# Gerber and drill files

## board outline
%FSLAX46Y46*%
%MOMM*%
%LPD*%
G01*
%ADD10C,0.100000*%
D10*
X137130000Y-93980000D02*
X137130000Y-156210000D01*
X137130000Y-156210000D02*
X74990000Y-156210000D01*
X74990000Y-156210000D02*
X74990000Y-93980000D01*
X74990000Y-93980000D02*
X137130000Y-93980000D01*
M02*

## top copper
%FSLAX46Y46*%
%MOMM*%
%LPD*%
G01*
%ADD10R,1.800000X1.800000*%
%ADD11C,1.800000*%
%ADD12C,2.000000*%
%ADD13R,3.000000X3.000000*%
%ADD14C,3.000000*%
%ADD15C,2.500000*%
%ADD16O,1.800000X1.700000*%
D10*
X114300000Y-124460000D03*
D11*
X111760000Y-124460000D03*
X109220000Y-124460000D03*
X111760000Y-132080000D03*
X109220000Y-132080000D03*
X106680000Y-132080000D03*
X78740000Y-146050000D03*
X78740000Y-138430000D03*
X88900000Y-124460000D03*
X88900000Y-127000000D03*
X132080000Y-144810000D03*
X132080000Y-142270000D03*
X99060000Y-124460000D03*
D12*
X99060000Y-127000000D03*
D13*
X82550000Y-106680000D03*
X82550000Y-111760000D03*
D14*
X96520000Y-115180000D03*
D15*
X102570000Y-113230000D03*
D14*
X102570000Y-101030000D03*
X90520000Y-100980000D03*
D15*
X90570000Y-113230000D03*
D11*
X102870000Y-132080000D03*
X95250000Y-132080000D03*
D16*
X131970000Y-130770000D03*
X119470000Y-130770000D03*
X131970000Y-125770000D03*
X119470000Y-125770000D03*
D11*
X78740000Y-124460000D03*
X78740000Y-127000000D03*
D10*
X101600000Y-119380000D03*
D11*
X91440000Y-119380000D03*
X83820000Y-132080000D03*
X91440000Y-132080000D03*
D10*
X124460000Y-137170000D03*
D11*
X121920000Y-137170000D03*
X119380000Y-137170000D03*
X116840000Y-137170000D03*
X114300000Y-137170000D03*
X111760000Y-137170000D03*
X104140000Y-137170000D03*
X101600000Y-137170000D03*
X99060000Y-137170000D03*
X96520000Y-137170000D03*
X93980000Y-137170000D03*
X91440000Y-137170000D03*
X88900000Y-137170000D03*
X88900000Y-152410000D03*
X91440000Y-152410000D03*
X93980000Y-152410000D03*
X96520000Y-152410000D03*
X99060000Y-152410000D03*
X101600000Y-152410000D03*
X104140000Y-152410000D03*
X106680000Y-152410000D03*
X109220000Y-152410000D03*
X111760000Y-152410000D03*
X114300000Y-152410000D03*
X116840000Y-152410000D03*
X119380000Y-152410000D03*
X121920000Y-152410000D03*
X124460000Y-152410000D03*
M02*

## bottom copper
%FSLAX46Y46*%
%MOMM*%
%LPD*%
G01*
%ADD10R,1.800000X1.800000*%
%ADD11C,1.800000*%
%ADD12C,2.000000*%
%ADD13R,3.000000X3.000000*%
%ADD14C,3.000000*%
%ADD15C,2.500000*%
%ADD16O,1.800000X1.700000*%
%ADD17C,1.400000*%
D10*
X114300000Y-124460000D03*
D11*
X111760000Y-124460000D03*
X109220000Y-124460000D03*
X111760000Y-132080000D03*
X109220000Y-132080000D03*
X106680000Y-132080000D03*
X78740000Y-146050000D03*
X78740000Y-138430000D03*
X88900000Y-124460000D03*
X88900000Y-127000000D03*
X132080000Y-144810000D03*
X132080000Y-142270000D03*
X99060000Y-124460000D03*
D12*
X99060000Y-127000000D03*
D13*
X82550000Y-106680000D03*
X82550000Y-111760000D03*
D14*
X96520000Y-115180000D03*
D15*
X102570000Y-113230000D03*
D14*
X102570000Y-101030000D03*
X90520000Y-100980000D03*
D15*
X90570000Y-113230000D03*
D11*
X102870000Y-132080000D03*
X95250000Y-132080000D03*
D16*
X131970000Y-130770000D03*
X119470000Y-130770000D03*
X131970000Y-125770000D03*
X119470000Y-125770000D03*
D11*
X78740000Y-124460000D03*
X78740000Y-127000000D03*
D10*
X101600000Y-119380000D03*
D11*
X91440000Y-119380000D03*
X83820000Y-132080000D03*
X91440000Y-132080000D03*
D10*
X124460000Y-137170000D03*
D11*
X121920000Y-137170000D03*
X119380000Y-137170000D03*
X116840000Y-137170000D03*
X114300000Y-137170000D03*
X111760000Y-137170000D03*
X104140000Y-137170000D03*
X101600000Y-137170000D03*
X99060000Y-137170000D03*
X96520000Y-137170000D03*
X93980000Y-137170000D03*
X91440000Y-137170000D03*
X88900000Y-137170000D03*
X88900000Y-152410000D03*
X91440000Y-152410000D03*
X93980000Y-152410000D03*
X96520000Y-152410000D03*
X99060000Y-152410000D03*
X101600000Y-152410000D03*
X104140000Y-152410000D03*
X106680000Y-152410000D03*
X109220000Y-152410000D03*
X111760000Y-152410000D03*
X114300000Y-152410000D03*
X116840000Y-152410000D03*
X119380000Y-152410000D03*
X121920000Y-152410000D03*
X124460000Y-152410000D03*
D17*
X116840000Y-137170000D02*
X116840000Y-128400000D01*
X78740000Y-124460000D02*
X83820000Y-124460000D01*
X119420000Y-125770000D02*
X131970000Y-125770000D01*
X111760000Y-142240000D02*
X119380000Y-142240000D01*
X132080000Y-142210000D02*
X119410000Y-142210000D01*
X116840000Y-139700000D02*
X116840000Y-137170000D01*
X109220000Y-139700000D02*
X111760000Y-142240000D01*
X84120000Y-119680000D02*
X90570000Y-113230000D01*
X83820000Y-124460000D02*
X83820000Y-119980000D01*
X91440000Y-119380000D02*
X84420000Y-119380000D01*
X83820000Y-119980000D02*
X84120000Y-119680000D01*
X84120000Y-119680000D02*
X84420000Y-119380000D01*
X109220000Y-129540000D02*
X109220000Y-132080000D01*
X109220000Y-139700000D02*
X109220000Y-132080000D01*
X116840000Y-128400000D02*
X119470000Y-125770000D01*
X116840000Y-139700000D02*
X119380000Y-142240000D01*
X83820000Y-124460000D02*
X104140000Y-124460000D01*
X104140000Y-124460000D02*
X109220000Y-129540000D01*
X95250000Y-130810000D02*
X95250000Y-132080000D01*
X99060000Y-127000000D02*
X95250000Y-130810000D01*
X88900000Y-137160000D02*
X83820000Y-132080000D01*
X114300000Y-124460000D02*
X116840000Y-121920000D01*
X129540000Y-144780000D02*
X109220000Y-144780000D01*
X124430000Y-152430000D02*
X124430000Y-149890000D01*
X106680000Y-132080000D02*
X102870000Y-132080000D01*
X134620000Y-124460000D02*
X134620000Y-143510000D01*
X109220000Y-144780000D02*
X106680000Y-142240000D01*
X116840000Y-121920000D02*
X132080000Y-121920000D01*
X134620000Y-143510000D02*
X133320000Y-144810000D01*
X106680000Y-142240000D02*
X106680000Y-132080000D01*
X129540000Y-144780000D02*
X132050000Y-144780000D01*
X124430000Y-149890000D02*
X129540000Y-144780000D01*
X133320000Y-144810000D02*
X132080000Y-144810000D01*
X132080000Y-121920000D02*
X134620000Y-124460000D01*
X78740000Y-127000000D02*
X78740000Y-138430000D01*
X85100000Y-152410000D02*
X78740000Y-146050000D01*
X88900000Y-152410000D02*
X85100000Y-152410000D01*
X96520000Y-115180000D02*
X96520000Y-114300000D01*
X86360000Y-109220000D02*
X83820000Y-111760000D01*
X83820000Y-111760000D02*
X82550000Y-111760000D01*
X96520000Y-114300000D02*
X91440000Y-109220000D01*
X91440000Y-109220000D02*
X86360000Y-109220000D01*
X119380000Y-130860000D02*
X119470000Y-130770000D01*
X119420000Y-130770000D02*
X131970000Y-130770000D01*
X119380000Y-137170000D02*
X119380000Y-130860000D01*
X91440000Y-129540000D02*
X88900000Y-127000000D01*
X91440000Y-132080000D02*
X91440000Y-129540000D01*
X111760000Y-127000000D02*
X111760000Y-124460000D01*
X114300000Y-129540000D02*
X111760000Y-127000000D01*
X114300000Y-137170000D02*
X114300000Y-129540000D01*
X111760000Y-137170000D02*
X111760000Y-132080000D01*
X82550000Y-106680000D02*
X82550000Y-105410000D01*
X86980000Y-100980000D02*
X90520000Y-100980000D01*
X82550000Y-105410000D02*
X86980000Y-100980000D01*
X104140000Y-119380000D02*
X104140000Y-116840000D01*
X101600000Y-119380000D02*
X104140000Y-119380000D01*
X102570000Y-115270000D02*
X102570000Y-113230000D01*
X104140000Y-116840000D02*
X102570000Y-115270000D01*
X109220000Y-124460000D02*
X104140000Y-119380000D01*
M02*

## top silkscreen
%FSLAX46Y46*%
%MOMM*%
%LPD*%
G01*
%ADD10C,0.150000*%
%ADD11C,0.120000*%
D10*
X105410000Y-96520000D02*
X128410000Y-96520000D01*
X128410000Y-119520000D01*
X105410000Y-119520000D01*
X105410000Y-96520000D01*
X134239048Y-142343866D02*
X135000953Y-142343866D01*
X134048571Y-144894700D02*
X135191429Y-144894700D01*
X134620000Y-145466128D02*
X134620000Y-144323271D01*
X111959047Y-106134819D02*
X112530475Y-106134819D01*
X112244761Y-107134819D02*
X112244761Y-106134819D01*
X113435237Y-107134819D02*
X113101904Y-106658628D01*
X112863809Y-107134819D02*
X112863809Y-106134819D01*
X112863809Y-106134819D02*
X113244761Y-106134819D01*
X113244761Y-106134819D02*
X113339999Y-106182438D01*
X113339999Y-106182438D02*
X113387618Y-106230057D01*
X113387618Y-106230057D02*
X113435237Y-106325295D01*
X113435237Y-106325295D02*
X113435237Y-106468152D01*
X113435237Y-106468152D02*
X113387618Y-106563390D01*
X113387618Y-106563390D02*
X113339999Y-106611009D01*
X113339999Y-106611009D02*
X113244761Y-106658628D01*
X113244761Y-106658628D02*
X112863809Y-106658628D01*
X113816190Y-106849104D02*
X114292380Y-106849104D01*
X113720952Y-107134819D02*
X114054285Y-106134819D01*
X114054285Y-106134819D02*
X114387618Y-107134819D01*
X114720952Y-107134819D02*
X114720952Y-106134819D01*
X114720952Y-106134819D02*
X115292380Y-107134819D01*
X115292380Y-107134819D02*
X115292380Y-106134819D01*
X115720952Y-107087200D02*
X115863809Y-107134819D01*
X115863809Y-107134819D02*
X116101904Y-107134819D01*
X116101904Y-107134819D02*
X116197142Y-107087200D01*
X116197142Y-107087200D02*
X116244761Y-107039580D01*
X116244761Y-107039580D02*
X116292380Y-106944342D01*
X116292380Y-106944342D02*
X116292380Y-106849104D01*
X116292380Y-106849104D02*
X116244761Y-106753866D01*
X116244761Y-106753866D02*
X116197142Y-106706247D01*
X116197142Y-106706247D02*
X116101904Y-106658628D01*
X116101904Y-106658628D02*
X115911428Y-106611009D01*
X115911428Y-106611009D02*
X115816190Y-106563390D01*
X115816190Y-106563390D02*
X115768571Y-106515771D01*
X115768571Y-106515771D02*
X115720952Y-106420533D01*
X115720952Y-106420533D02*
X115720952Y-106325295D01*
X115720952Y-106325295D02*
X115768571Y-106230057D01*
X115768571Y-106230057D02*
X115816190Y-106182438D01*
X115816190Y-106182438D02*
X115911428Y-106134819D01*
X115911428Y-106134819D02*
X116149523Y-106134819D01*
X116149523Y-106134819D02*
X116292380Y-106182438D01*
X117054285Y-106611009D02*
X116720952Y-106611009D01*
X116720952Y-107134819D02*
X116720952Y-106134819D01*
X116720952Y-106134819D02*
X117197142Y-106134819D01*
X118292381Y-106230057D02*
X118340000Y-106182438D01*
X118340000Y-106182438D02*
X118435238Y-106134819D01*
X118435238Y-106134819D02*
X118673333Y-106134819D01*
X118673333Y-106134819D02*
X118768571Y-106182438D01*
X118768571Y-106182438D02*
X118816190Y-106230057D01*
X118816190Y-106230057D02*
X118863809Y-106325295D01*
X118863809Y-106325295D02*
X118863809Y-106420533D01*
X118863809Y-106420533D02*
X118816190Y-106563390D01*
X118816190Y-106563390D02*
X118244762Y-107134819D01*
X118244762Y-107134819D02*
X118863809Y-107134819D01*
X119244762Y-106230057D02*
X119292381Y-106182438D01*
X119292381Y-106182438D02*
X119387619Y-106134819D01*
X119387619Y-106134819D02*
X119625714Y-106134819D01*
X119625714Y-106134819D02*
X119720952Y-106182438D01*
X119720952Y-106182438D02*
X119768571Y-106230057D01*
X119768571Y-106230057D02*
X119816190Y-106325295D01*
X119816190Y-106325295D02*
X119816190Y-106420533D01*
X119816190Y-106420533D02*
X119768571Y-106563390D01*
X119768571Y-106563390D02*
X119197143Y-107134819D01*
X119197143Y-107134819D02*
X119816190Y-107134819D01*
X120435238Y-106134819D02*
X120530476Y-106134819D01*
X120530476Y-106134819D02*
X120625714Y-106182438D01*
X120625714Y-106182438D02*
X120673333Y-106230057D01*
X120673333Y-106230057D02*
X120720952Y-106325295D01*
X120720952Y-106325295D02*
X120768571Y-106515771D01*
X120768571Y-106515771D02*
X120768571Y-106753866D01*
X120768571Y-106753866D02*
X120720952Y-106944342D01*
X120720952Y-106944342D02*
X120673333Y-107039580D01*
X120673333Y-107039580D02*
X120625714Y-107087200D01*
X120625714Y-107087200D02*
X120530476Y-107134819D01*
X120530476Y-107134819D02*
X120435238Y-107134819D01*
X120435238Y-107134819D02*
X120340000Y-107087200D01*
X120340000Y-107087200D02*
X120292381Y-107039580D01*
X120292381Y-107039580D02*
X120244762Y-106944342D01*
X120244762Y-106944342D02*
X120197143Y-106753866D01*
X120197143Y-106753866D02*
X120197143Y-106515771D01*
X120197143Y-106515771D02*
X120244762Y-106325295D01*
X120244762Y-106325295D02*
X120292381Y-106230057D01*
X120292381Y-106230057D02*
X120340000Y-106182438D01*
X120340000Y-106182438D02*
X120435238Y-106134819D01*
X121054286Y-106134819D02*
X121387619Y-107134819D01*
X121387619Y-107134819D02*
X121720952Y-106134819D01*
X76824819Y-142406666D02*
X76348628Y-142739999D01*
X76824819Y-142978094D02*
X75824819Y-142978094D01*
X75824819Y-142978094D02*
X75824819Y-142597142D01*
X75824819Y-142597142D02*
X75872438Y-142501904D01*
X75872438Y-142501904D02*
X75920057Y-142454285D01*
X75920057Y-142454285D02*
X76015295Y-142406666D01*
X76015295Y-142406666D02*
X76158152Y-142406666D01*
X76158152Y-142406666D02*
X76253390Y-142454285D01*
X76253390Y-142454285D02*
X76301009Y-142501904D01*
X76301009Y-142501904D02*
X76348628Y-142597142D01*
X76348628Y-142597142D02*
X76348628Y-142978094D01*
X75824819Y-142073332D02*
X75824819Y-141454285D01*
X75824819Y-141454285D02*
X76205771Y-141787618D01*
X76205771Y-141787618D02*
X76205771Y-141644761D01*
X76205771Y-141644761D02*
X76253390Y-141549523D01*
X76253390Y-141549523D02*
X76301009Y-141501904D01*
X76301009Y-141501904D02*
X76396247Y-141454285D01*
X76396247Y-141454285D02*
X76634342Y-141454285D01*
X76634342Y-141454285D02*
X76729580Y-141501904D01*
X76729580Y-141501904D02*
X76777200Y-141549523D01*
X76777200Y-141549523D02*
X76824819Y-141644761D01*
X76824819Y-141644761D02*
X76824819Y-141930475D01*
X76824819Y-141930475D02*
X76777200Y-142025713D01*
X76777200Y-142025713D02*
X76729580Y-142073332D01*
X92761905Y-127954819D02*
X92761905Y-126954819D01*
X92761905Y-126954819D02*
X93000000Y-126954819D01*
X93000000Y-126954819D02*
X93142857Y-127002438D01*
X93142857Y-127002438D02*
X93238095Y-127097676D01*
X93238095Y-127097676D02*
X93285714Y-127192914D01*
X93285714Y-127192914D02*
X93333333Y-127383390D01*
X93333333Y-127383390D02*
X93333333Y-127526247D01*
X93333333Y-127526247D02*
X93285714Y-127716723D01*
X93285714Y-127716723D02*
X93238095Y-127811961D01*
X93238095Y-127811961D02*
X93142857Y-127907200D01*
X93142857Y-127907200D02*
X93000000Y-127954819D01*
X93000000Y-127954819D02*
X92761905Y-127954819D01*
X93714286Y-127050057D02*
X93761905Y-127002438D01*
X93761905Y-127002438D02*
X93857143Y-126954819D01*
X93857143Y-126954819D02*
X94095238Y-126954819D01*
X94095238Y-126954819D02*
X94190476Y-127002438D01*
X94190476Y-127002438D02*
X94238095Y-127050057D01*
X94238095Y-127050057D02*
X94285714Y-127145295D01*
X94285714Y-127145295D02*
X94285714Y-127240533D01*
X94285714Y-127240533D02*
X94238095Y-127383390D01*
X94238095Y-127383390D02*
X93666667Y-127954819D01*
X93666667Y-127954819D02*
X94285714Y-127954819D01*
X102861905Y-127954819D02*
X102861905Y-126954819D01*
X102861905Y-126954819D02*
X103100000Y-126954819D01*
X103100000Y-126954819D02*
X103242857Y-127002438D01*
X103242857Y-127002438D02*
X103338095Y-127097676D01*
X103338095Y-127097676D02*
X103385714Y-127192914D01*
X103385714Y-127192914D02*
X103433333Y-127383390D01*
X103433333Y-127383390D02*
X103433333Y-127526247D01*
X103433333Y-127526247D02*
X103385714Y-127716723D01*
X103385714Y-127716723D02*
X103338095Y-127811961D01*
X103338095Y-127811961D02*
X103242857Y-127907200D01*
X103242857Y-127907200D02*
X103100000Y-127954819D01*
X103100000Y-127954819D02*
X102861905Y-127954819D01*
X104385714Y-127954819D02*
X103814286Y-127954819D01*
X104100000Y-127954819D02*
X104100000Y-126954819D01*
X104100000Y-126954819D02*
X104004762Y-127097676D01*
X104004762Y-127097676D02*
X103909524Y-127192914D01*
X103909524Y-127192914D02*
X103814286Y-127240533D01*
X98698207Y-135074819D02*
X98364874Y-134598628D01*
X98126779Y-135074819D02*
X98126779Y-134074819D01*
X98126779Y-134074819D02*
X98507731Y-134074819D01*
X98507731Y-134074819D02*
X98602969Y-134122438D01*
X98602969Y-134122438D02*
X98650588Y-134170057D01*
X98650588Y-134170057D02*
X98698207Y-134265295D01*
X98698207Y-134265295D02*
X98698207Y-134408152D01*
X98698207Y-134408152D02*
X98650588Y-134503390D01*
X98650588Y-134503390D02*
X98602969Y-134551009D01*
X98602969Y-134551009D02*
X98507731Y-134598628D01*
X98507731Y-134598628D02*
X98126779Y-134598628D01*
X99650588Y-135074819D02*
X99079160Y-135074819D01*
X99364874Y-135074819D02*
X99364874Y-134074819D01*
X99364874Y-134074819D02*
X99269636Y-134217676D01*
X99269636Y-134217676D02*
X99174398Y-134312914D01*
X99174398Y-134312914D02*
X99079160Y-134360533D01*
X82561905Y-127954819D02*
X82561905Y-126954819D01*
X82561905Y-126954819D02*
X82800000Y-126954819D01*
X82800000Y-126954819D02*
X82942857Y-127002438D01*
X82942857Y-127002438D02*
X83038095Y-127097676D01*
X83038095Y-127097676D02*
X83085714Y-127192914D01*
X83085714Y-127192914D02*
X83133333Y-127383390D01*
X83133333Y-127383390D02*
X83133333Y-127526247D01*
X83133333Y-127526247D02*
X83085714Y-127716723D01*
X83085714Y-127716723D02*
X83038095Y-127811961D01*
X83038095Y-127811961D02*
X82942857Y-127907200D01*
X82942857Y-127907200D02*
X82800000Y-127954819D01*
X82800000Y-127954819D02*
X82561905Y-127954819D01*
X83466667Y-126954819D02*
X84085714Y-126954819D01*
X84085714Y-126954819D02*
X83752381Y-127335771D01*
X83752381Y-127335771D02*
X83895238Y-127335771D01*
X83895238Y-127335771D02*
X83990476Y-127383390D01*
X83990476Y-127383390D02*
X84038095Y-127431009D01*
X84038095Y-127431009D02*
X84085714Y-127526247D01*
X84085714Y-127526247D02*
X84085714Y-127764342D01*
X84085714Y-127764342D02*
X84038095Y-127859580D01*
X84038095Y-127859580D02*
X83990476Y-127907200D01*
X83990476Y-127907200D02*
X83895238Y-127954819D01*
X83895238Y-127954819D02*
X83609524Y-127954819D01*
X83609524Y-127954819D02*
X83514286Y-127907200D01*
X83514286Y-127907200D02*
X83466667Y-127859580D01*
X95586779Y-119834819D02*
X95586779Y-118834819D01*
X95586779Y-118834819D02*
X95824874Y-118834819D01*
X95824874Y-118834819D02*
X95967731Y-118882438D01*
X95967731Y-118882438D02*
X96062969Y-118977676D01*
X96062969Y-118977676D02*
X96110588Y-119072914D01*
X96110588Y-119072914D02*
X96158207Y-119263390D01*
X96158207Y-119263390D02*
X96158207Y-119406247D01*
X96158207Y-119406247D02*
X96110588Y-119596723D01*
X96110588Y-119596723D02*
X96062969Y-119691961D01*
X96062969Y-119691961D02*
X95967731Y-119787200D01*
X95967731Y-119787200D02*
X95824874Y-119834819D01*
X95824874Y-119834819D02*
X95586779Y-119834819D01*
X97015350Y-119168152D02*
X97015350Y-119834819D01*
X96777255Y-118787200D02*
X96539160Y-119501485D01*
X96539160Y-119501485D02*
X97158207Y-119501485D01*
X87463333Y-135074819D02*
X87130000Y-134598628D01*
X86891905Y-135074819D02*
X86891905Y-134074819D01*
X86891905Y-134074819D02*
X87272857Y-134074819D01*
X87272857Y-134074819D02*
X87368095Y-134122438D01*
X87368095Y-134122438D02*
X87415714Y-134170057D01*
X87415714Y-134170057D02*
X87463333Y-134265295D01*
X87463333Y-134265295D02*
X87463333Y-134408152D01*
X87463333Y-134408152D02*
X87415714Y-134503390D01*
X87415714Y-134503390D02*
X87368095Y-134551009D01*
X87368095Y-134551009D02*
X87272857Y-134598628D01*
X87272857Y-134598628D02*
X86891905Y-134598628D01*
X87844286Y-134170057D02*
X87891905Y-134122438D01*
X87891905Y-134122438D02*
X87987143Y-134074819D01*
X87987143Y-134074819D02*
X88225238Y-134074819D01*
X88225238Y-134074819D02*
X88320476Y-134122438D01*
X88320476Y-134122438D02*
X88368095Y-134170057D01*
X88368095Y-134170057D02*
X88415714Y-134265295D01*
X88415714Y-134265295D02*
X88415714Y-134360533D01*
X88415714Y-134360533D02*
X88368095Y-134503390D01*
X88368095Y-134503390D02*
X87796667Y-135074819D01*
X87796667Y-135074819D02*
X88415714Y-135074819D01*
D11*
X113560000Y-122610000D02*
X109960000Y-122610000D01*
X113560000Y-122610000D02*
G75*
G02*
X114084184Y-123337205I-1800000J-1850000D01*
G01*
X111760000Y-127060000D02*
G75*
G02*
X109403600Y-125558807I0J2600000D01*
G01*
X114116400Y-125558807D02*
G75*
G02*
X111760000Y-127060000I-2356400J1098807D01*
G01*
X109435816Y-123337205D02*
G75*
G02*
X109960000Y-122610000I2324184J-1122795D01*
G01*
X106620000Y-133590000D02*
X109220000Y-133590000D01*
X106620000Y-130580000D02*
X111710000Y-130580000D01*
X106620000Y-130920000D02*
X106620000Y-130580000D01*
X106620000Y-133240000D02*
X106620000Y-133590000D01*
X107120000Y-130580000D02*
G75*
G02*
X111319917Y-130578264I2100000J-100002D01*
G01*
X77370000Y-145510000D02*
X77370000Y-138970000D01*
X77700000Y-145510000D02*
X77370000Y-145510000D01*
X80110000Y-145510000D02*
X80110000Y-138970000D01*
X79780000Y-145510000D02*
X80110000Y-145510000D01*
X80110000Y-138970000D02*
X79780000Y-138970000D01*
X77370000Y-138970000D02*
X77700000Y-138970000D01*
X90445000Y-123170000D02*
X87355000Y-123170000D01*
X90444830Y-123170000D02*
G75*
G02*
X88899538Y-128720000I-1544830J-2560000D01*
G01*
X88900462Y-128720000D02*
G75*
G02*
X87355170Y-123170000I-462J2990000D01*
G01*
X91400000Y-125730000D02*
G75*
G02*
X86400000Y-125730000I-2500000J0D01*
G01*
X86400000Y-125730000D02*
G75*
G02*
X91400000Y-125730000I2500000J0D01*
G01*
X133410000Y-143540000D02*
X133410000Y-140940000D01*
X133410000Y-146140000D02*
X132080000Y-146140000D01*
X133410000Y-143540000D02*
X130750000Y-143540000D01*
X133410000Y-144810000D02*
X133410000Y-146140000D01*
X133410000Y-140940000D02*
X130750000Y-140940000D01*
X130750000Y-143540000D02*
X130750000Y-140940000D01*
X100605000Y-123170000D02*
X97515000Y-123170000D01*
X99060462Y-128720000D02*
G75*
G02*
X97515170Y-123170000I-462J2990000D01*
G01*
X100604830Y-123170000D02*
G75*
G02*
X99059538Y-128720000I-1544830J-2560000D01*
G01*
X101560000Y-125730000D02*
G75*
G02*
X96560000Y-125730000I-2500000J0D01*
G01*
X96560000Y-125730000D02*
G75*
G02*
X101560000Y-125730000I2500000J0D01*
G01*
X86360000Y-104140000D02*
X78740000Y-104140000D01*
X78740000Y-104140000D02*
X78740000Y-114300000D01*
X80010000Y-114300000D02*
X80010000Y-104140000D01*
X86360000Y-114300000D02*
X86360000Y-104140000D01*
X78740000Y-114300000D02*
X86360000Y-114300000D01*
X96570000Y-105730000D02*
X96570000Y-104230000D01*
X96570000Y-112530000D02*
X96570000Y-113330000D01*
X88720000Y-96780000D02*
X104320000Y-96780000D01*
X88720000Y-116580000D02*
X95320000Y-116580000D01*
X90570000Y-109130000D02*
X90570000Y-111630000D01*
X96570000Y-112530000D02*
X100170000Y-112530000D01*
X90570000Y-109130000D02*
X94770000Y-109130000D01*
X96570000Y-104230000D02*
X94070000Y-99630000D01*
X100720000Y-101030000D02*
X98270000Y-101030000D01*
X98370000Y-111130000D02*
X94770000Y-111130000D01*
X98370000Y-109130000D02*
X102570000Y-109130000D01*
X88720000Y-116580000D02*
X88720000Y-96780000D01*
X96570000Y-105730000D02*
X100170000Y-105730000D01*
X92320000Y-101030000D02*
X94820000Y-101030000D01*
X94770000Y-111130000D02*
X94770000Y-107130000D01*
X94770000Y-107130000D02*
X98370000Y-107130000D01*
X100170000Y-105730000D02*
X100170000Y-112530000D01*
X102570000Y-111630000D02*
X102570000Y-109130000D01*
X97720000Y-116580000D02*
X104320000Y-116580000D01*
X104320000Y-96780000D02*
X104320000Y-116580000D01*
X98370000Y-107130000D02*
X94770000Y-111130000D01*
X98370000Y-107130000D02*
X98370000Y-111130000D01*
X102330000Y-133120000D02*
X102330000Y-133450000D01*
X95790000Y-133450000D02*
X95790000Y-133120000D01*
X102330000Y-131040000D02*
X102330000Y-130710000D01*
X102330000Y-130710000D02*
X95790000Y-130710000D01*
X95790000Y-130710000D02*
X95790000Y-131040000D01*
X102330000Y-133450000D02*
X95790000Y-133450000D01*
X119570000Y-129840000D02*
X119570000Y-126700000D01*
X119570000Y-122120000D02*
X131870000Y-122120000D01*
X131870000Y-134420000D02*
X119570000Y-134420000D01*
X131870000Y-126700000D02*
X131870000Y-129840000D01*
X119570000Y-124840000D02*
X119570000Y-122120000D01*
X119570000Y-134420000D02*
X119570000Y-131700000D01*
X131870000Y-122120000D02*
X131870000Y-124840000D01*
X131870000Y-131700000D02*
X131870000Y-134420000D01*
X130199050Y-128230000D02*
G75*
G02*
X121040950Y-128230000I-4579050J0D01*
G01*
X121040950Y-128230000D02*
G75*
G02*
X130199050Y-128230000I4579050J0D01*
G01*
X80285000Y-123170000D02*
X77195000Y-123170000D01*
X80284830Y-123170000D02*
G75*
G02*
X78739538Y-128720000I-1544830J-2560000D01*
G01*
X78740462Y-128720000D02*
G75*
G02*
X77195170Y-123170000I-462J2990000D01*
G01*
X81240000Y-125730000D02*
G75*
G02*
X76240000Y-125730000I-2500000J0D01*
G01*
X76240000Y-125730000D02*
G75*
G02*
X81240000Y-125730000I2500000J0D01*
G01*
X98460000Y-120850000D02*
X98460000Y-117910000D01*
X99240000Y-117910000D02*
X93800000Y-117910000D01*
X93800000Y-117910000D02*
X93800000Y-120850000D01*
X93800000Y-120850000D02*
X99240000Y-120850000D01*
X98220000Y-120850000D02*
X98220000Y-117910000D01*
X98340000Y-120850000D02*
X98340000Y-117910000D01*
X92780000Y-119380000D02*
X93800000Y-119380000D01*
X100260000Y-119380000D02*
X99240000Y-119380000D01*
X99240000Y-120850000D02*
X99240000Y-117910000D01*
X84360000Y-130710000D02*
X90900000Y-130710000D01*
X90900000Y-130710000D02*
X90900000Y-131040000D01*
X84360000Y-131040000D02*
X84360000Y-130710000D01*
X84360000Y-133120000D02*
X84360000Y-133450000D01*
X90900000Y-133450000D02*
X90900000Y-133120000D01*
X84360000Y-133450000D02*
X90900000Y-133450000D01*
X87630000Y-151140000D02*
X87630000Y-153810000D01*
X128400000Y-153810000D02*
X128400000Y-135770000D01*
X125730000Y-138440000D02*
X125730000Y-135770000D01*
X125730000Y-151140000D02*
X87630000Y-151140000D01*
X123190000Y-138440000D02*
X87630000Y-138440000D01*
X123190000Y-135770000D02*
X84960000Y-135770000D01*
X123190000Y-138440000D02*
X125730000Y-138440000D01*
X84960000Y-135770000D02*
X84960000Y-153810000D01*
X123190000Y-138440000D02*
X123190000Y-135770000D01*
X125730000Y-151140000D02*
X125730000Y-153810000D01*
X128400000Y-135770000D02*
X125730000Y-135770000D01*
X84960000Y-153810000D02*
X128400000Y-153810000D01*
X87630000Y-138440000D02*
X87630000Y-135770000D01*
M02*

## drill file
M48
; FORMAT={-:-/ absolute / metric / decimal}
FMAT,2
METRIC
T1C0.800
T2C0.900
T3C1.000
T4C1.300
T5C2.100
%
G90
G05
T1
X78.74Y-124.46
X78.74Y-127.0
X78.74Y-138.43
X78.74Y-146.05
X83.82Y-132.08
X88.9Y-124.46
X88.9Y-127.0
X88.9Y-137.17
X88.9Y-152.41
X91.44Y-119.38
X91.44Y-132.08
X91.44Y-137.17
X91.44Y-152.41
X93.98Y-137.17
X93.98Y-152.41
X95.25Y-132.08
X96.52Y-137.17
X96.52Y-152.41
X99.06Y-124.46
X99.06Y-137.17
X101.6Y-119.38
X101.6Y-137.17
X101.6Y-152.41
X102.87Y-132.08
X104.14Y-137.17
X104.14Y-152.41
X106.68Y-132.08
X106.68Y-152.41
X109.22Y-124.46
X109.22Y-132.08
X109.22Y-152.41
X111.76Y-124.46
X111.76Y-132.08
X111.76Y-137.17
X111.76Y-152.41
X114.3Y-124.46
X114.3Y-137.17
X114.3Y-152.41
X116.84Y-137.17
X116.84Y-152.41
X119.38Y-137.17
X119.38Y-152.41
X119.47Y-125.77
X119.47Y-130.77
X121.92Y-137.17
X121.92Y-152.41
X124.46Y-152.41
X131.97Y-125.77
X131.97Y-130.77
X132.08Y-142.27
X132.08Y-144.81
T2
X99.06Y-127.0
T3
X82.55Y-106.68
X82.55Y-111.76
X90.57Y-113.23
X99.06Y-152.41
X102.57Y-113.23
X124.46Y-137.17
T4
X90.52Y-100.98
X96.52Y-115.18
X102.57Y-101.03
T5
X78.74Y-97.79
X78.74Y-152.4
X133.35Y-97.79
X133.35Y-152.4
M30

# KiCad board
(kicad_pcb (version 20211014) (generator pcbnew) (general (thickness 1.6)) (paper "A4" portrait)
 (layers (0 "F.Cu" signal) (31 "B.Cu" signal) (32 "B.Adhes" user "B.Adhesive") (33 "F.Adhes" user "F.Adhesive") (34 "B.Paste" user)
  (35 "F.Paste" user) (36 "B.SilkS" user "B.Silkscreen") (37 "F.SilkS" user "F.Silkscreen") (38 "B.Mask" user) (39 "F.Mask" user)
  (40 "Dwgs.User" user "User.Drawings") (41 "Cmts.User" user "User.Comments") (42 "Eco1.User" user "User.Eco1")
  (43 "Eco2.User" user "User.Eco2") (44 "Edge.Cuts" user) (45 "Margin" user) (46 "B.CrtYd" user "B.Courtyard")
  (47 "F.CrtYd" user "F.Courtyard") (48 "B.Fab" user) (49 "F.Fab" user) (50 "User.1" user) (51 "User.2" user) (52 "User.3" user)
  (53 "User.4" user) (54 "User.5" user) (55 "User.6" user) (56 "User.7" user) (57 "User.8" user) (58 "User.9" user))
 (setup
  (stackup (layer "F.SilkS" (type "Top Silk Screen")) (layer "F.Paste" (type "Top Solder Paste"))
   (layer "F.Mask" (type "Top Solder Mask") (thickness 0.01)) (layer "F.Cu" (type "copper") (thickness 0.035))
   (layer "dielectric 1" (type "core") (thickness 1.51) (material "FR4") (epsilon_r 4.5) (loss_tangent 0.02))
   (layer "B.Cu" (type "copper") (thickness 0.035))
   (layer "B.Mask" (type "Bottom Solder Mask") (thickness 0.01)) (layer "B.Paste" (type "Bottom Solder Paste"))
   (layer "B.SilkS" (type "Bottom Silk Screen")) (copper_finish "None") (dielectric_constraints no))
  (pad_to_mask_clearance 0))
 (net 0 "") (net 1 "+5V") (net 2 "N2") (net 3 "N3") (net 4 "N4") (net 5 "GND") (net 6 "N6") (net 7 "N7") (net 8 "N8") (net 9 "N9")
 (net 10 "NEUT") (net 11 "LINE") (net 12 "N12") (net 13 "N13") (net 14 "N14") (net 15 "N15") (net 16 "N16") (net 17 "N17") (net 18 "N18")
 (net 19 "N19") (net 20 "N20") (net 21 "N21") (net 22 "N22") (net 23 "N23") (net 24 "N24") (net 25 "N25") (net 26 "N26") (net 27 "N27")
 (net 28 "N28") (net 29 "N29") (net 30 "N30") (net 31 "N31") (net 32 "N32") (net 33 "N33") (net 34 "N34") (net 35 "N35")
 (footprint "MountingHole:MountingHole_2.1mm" (layer "F.Cu") (at 133.35 97.79)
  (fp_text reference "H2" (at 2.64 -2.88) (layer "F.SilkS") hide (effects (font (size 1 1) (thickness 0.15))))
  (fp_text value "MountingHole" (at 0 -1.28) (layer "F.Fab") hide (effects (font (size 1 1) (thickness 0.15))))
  (pad "" np_thru_hole circle (at 0 0) (size 2.1 2.1) (drill 2.1) (layers *.Cu *.Mask)))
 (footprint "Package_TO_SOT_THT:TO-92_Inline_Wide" (layer "F.Cu") (at 114.3 124.46 180)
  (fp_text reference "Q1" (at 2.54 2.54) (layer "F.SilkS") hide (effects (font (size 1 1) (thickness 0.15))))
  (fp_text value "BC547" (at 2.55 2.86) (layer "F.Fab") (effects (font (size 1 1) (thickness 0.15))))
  (fp_line (start 0.74 1.85) (end 4.34 1.85) (layer "F.SilkS") (width 0.12))
  (fp_arc (start 0.74 1.85) (mid 0.446097 1.509328) (end 0.215816 1.122795) (layer "F.SilkS") (width 0.12))
  (fp_arc (start 2.54 -2.6) (mid 3.936979 -2.192818) (end 4.8964 -1.098807) (layer "F.SilkS") (width 0.12))
  (fp_arc (start 0.1836 -1.098807) (mid 1.143021 -2.192817) (end 2.54 -2.6) (layer "F.SilkS") (width 0.12))
  (fp_arc (start 4.864184 1.122795) (mid 4.633903 1.509328) (end 4.34 1.85) (layer "F.SilkS") (width 0.12))
  (pad "1" thru_hole rect (at 0 0 180) (size 1.8 1.8) (drill 0.8) (layers *.Cu *.Mask) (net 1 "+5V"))
  (pad "2" thru_hole circle (at 2.54 0 180) (size 1.8 1.8) (drill 0.8) (layers *.Cu *.Mask) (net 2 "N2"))
  (pad "3" thru_hole circle (at 5.08 0 180) (size 1.8 1.8) (drill 0.8) (layers *.Cu *.Mask) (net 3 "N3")))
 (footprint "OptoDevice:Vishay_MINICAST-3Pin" (layer "F.Cu") (at 111.76 132.08 180)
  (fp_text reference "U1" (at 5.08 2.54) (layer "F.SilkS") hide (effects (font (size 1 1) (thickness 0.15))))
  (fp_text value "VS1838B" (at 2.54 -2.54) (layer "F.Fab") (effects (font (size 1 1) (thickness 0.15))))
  (fp_line (start 5.14 -1.51) (end 2.54 -1.51) (layer "F.SilkS") (width 0.12))
  (fp_line (start 5.14 1.5) (end 0.05 1.5) (layer "F.SilkS") (width 0.12))
  (fp_line (start 5.14 1.16) (end 5.14 1.5) (layer "F.SilkS") (width 0.12))
  (fp_line (start 5.14 -1.16) (end 5.14 -1.51) (layer "F.SilkS") (width 0.12))
  (fp_arc (start 4.64 1.5) (mid 2.540869 3.502378) (end 0.440083 1.501736) (layer "F.SilkS") (width 0.12))
  (pad "1" thru_hole circle (at 0 0 180) (size 1.8 1.8) (drill 0.8) (layers *.Cu *.Mask) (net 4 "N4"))
  (pad "2" thru_hole circle (at 2.54 0 180) (size 1.8 1.8) (drill 0.8) (layers *.Cu *.Mask) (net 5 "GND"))
  (pad "3" thru_hole circle (at 5.08 0 180) (size 1.8 1.8) (drill 0.8) (layers *.Cu *.Mask) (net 1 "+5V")))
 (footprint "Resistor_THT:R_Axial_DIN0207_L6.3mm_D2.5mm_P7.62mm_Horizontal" (layer "F.Cu") (at 78.74 146.05 90)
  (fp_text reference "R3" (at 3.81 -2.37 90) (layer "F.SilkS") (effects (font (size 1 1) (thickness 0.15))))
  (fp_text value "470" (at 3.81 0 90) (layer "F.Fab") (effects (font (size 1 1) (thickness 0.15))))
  (fp_line (start 0.54 -1.37) (end 7.08 -1.37) (layer "F.SilkS") (width 0.12))
  (fp_line (start 0.54 -1.04) (end 0.54 -1.37) (layer "F.SilkS") (width 0.12))
  (fp_line (start 0.54 1.37) (end 7.08 1.37) (layer "F.SilkS") (width 0.12))
  (fp_line (start 0.54 1.04) (end 0.54 1.37) (layer "F.SilkS") (width 0.12))
  (fp_line (start 7.08 1.37) (end 7.08 1.04) (layer "F.SilkS") (width 0.12))
  (fp_line (start 7.08 -1.37) (end 7.08 -1.04) (layer "F.SilkS") (width 0.12))
  (pad "1" thru_hole circle (at 0 0 90) (size 1.8 1.8) (drill 0.8) (layers *.Cu *.Mask) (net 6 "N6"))
  (pad "2" thru_hole circle (at 7.62 0 90) (size 1.8 1.8) (drill 0.8) (layers *.Cu *.Mask) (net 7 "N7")))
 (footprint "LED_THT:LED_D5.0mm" (layer "F.Cu") (at 88.9 124.46 -90)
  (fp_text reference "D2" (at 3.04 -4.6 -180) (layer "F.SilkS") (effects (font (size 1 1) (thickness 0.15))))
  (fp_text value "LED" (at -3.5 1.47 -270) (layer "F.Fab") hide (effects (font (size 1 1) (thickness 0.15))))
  (fp_line (start -1.29 -1.545) (end -1.29 1.545) (layer "F.SilkS") (width 0.12))
  (fp_arc (start -1.29 -1.54483) (mid 2.072002 -2.880433) (end 4.26 0.000462) (layer "F.SilkS") (width 0.12))
  (fp_arc (start 4.26 -0.000462) (mid 2.072002 2.880433) (end -1.29 1.54483) (layer "F.SilkS") (width 0.12))
  (fp_circle (center 1.27 0) (end 3.77 0) (layer "F.SilkS") (width 0.12) (fill none))
  (pad "1" thru_hole circle (at 0 0 270) (size 1.8 1.8) (drill 0.8) (layers *.Cu *.Mask) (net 5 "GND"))
  (pad "2" thru_hole circle (at 2.54 0 270) (size 1.8 1.8) (drill 0.8) (layers *.Cu *.Mask) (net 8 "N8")))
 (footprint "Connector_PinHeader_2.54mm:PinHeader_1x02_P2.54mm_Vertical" (layer "F.Cu") (at 132.08 144.81 180)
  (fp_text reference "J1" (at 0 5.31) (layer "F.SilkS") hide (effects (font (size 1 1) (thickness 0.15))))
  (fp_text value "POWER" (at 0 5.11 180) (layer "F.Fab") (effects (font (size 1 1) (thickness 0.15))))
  (fp_line (start -1.33 1.27) (end -1.33 3.87) (layer "F.SilkS") (width 0.12))
  (fp_line (start -1.33 -1.33) (end 0 -1.33) (layer "F.SilkS") (width 0.12))
  (fp_line (start -1.33 1.27) (end 1.33 1.27) (layer "F.SilkS") (width 0.12))
  (fp_line (start -1.33 0) (end -1.33 -1.33) (layer "F.SilkS") (width 0.12))
  (fp_line (start -1.33 3.87) (end 1.33 3.87) (layer "F.SilkS") (width 0.12))
  (fp_line (start 1.33 1.27) (end 1.33 3.87) (layer "F.SilkS") (width 0.12))
  (pad "1" thru_hole circle (at 0 0 180) (size 1.8 1.8) (drill 0.8) (layers *.Cu *.Mask) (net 1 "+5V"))
  (pad "2" thru_hole circle (at 0 2.54 180) (size 1.8 1.8) (drill 0.8) (layers *.Cu *.Mask) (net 5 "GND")))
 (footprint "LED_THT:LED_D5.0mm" (layer "F.Cu") (at 99.06 124.46 -90)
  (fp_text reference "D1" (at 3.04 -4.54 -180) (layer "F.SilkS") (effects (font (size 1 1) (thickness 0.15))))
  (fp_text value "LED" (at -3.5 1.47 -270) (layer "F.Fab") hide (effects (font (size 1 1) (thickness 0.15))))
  (fp_line (start -1.29 -1.545) (end -1.29 1.545) (layer "F.SilkS") (width 0.12))
  (fp_arc (start 4.26 -0.000462) (mid 2.072002 2.880433) (end -1.29 1.54483) (layer "F.SilkS") (width 0.12))
  (fp_arc (start -1.29 -1.54483) (mid 2.072002 -2.880433) (end 4.26 0.000462) (layer "F.SilkS") (width 0.12))
  (fp_circle (center 1.27 0) (end 3.77 0) (layer "F.SilkS") (width 0.12) (fill none))
  (pad "1" thru_hole circle (at 0 0 270) (size 1.8 1.8) (drill 0.8) (layers *.Cu *.Mask) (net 5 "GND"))
  (pad "2" thru_hole circle (at 2.54 0 270) (size 2 2) (drill 0.9) (layers *.Cu *.Mask) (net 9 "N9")))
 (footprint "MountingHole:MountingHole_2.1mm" (layer "F.Cu") (at 133.35 152.4)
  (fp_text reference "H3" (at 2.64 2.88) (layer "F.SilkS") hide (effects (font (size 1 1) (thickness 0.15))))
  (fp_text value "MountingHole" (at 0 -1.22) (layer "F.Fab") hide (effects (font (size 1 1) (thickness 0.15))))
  (pad "" np_thru_hole circle (at 0 0) (size 2.1 2.1) (drill 2.1) (layers *.Cu *.Mask)))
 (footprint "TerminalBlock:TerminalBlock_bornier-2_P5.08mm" (layer "F.Cu") (at 82.55 106.68 -90)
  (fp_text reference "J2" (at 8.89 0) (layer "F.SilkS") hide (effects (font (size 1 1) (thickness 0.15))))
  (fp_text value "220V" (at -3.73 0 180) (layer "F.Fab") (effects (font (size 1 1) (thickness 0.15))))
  (fp_line (start -2.54 -3.81) (end -2.54 3.81) (layer "F.SilkS") (width 0.12))
  (fp_line (start -2.54 3.81) (end 7.62 3.81) (layer "F.SilkS") (width 0.12))
  (fp_line (start 7.62 2.54) (end -2.54 2.54) (layer "F.SilkS") (width 0.12))
  (fp_line (start 7.62 -3.81) (end -2.54 -3.81) (layer "F.SilkS") (width 0.12))
  (fp_line (start 7.62 3.81) (end 7.62 -3.81) (layer "F.SilkS") (width 0.12))
  (pad "1" thru_hole rect (at 0 0 270) (size 3 3) (drill 1) (layers *.Cu *.Mask) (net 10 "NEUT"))
  (pad "2" thru_hole rect (at 5.08 0 270) (size 3 3) (drill 1) (layers *.Cu *.Mask) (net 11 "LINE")))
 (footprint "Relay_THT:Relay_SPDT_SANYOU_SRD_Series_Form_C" (layer "F.Cu") (at 96.52 115.18 90)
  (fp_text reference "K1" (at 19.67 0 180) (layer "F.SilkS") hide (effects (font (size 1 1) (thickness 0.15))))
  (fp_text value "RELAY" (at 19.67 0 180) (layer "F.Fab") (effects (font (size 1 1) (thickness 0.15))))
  (fp_line (start 9.45 0.05) (end 10.95 0.05) (layer "F.SilkS") (width 0.12))
  (fp_line (start 2.65 0.05) (end 1.85 0.05) (layer "F.SilkS") (width 0.12))
  (fp_line (start 18.4 -7.8) (end 18.4 7.8) (layer "F.SilkS") (width 0.12))
  (fp_line (start -1.4 -7.8) (end -1.4 -1.2) (layer "F.SilkS") (width 0.12))
  (fp_line (start 6.05 -5.95) (end 3.55 -5.95) (layer "F.SilkS") (width 0.12))
  (fp_line (start 2.65 0.05) (end 2.65 3.65) (layer "F.SilkS") (width 0.12))
  (fp_line (start 6.05 -5.95) (end 6.05 -1.75) (layer "F.SilkS") (width 0.12))
  (fp_line (start 10.95 0.05) (end 15.55 -2.45) (layer "F.SilkS") (width 0.12))
  (fp_line (start 14.15 4.2) (end 14.15 1.75) (layer "F.SilkS") (width 0.12))
  (fp_line (start 4.05 1.85) (end 4.05 -1.75) (layer "F.SilkS") (width 0.12))
  (fp_line (start 6.05 1.85) (end 6.05 6.05) (layer "F.SilkS") (width 0.12))
  (fp_line (start -1.4 -7.8) (end 18.4 -7.8) (layer "F.SilkS") (width 0.12))
  (fp_line (start 9.45 0.05) (end 9.45 3.65) (layer "F.SilkS") (width 0.12))
  (fp_line (start 14.15 -4.2) (end 14.15 -1.7) (layer "F.SilkS") (width 0.12))
  (fp_line (start 4.05 -1.75) (end 8.05 -1.75) (layer "F.SilkS") (width 0.12))
  (fp_line (start 8.05 -1.75) (end 8.05 1.85) (layer "F.SilkS") (width 0.12))
  (fp_line (start 9.45 3.65) (end 2.65 3.65) (layer "F.SilkS") (width 0.12))
  (fp_line (start 3.55 6.05) (end 6.05 6.05) (layer "F.SilkS") (width 0.12))
  (fp_line (start -1.4 1.2) (end -1.4 7.8) (layer "F.SilkS") (width 0.12))
  (fp_line (start 18.4 7.8) (end -1.4 7.8) (layer "F.SilkS") (width 0.12))
  (fp_line (start 8.05 1.85) (end 4.05 -1.75) (layer "F.SilkS") (width 0.12))
  (fp_line (start 8.05 1.85) (end 4.05 1.85) (layer "F.SilkS") (width 0.12))
  (pad "1" thru_hole circle (at 0 0 180) (size 3 3) (drill 1.3) (layers *.Cu *.Mask) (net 11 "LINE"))
  (pad "2" thru_hole circle (at 1.95 6.05 180) (size 2.5 2.5) (drill 1) (layers *.Cu *.Mask) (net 3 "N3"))
  (pad "3" thru_hole circle (at 14.15 6.05 180) (size 3 3) (drill 1.3) (layers *.Cu *.Mask) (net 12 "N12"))
  (pad "4" thru_hole circle (at 14.2 -6 180) (size 3 3) (drill 1.3) (layers *.Cu *.Mask) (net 10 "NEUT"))
  (pad "5" thru_hole circle (at 1.95 -5.95 180) (size 2.5 2.5) (drill 1) (layers *.Cu *.Mask) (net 5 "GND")))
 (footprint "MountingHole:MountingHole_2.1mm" (layer "F.Cu") (at 78.74 152.4)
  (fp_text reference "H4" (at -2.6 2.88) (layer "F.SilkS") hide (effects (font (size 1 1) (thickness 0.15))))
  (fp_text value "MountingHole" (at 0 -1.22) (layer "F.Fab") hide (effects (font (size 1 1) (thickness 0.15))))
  (pad "" np_thru_hole circle (at 0 0) (size 2.1 2.1) (drill 2.1) (layers F&B.Cu *.Mask)))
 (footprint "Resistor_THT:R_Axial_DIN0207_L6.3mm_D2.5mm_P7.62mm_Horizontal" (layer "F.Cu") (at 102.87 132.08 180)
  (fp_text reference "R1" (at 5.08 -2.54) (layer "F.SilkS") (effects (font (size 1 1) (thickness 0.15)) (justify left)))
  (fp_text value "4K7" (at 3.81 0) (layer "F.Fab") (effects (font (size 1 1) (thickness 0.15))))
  (fp_line (start 0.54 -1.04) (end 0.54 -1.37) (layer "F.SilkS") (width 0.12))
  (fp_line (start 7.08 -1.37) (end 7.08 -1.04) (layer "F.SilkS") (width 0.12))
  (fp_line (start 0.54 1.04) (end 0.54 1.37) (layer "F.SilkS") (width 0.12))
  (fp_line (start 0.54 1.37) (end 7.08 1.37) (layer "F.SilkS") (width 0.12))
  (fp_line (start 7.08 1.37) (end 7.08 1.04) (layer "F.SilkS") (width 0.12))
  (fp_line (start 0.54 -1.37) (end 7.08 -1.37) (layer "F.SilkS") (width 0.12))
  (pad "1" thru_hole circle (at 0 0 180) (size 1.8 1.8) (drill 0.8) (layers *.Cu *.Mask) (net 1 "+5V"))
  (pad "2" thru_hole circle (at 7.62 0 180) (size 1.8 1.8) (drill 0.8) (layers *.Cu *.Mask) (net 9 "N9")))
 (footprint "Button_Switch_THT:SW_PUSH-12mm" (layer "F.Cu") (at 131.97 130.77 180)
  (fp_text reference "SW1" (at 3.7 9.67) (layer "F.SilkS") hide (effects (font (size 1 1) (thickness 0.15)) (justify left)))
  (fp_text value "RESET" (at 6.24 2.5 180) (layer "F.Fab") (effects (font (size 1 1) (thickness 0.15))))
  (fp_line (start 12.4 0.93) (end 12.4 4.07) (layer "F.SilkS") (width 0.12))
  (fp_line (start 12.4 8.65) (end 0.1 8.65) (layer "F.SilkS") (width 0.12))
  (fp_line (start 0.1 -3.65) (end 12.4 -3.65) (layer "F.SilkS") (width 0.12))
  (fp_line (start 0.1 4.07) (end 0.1 0.93) (layer "F.SilkS") (width 0.12))
  (fp_line (start 12.4 5.93) (end 12.4 8.65) (layer "F.SilkS") (width 0.12))
  (fp_line (start 12.4 -3.65) (end 12.4 -0.93) (layer "F.SilkS") (width 0.12))
  (fp_line (start 0.1 8.65) (end 0.1 5.93) (layer "F.SilkS") (width 0.12))
  (fp_line (start 0.1 -0.93) (end 0.1 -3.65) (layer "F.SilkS") (width 0.12))
  (fp_circle (center 6.35 2.54) (end 10.16 5.08) (layer "F.SilkS") (width 0.12) (fill none))
  (pad "1" thru_hole oval (at 0 0 180) (size 1.8 1.7) (drill 0.8) (layers *.Cu *.Mask) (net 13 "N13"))
  (pad "1" thru_hole oval (at 12.5 0 180) (size 1.8 1.7) (drill 0.8) (layers *.Cu *.Mask) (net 13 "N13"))
  (pad "2" thru_hole oval (at 0 5 180) (size 1.8 1.7) (drill 0.8) (layers *.Cu *.Mask) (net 5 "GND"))
  (pad "2" thru_hole oval (at 12.5 5 180) (size 1.8 1.7) (drill 0.8) (layers *.Cu *.Mask) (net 5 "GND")))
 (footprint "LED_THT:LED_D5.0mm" (layer "F.Cu") (at 78.74 124.46 -90)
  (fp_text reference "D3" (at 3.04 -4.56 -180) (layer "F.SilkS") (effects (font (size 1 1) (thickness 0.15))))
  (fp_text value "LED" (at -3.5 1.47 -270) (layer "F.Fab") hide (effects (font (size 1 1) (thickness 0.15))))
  (fp_line (start -1.29 -1.545) (end -1.29 1.545) (layer "F.SilkS") (width 0.12))
  (fp_arc (start -1.29 -1.54483) (mid 2.072002 -2.880433) (end 4.26 0.000462) (layer "F.SilkS") (width 0.12))
  (fp_arc (start 4.26 -0.000462) (mid 2.072002 2.880433) (end -1.29 1.54483) (layer "F.SilkS") (width 0.12))
  (fp_circle (center 1.27 0) (end 3.77 0) (layer "F.SilkS") (width 0.12) (fill none))
  (pad "1" thru_hole circle (at 0 0 270) (size 1.8 1.8) (drill 0.8) (layers *.Cu *.Mask) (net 5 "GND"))
  (pad "2" thru_hole circle (at 2.54 0 270) (size 1.8 1.8) (drill 0.8) (layers *.Cu *.Mask) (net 7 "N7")))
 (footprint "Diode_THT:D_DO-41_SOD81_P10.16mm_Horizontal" (layer "F.Cu") (at 101.6 119.38 180)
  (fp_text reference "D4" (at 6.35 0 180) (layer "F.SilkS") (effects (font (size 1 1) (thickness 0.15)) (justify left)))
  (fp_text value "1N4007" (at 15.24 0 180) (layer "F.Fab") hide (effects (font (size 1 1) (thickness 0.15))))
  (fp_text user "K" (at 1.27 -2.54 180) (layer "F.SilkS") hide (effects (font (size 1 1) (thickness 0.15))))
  (fp_line (start 3.14 -1.47) (end 3.14 1.47) (layer "F.SilkS") (width 0.12))
  (fp_line (start 2.36 1.47) (end 7.8 1.47) (layer "F.SilkS") (width 0.12))
  (fp_line (start 7.8 1.47) (end 7.8 -1.47) (layer "F.SilkS") (width 0.12))
  (fp_line (start 7.8 -1.47) (end 2.36 -1.47) (layer "F.SilkS") (width 0.12))
  (fp_line (start 3.38 -1.47) (end 3.38 1.47) (layer "F.SilkS") (width 0.12))
  (fp_line (start 3.26 -1.47) (end 3.26 1.47) (layer "F.SilkS") (width 0.12))
  (fp_line (start 8.82 0) (end 7.8 0) (layer "F.SilkS") (width 0.12))
  (fp_line (start 1.34 0) (end 2.36 0) (layer "F.SilkS") (width 0.12))
  (fp_line (start 2.36 -1.47) (end 2.36 1.47) (layer "F.SilkS") (width 0.12))
  (pad "1" thru_hole rect (at 0 0 180) (size 1.8 1.8) (drill 0.8) (layers *.Cu *.Mask) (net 3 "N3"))
  (pad "2" thru_hole circle (at 10.16 0 180) (size 1.8 1.8) (drill 0.8) (layers *.Cu *.Mask) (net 5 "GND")))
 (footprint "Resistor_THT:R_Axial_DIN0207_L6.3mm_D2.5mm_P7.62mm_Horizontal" (layer "F.Cu") (at 83.82 132.08)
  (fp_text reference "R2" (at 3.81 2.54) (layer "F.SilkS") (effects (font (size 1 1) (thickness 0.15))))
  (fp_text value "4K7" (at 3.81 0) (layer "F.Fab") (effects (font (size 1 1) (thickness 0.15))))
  (fp_line (start 0.54 -1.37) (end 7.08 -1.37) (layer "F.SilkS") (width 0.12))
  (fp_line (start 7.08 -1.37) (end 7.08 -1.04) (layer "F.SilkS") (width 0.12))
  (fp_line (start 0.54 -1.04) (end 0.54 -1.37) (layer "F.SilkS") (width 0.12))
  (fp_line (start 0.54 1.04) (end 0.54 1.37) (layer "F.SilkS") (width 0.12))
  (fp_line (start 7.08 1.37) (end 7.08 1.04) (layer "F.SilkS") (width 0.12))
  (fp_line (start 0.54 1.37) (end 7.08 1.37) (layer "F.SilkS") (width 0.12))
  (pad "1" thru_hole circle (at 0 0) (size 1.8 1.8) (drill 0.8) (layers *.Cu *.Mask) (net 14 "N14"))
  (pad "2" thru_hole circle (at 7.62 0) (size 1.8 1.8) (drill 0.8) (layers *.Cu *.Mask) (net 8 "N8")))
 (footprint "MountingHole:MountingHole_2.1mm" (layer "F.Cu") (at 78.74 97.79)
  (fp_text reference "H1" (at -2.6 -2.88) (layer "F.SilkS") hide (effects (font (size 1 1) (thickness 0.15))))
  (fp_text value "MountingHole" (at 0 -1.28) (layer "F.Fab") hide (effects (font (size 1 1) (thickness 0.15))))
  (pad "" np_thru_hole circle (at 0 0) (size 2.1 2.1) (drill 2.1) (layers *.Cu *.Mask)))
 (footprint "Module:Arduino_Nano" (layer "F.Cu") (at 124.46 137.17 -90)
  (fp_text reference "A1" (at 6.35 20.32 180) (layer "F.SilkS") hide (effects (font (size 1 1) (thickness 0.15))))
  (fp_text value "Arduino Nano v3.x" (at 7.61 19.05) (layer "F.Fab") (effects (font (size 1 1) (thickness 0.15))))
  (fp_line (start 13.97 36.83) (end 16.64 36.83) (layer "F.SilkS") (width 0.12))
  (fp_line (start 16.64 -3.94) (end -1.4 -3.94) (layer "F.SilkS") (width 0.12))
  (fp_line (start 1.27 -1.27) (end -1.4 -1.27) (layer "F.SilkS") (width 0.12))
  (fp_line (start 13.97 -1.27) (end 13.97 36.83) (layer "F.SilkS") (width 0.12))
  (fp_line (start 1.27 1.27) (end 1.27 36.83) (layer "F.SilkS") (width 0.12))
  (fp_line (start -1.4 1.27) (end -1.4 39.5) (layer "F.SilkS") (width 0.12))
  (fp_line (start 1.27 1.27) (end 1.27 -1.27) (layer "F.SilkS") (width 0.12))
  (fp_line (start -1.4 39.5) (end 16.64 39.5) (layer "F.SilkS") (width 0.12))
  (fp_line (start 1.27 1.27) (end -1.4 1.27) (layer "F.SilkS") (width 0.12))
  (fp_line (start 13.97 -1.27) (end 16.64 -1.27) (layer "F.SilkS") (width 0.12))
  (fp_line (start -1.4 -3.94) (end -1.4 -1.27) (layer "F.SilkS") (width 0.12))
  (fp_line (start 16.64 39.5) (end 16.64 -3.94) (layer "F.SilkS") (width 0.12))
  (fp_line (start 1.27 36.83) (end -1.4 36.83) (layer "F.SilkS") (width 0.12))
  (pad "1" thru_hole rect (at 0 0 270) (size 1.8 1.8) (drill 1) (layers *.Cu *.Mask) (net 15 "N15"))
  (pad "2" thru_hole circle (at 0 2.54 270) (size 1.8 1.8) (drill 0.8) (layers *.Cu *.Mask) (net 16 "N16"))
  (pad "3" thru_hole circle (at 0 5.08 270) (size 1.8 1.8) (drill 0.8) (layers *.Cu *.Mask) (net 13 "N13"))
  (pad "4" thru_hole circle (at 0 7.62 270) (size 1.8 1.8) (drill 0.8) (layers *.Cu *.Mask) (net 5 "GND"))
  (pad "5" thru_hole circle (at 0 10.16 270) (size 1.8 1.8) (drill 0.8) (layers *.Cu *.Mask) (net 2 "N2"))
  (pad "6" thru_hole circle (at 0 12.7 270) (size 1.8 1.8) (drill 0.8) (layers *.Cu *.Mask) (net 4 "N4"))
  (pad "9" thru_hole circle (at 0 20.32 270) (size 1.8 1.8) (drill 0.8) (layers *.Cu *.Mask) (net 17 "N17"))
  (pad "10" thru_hole circle (at 0 22.86 270) (size 1.8 1.8) (drill 0.8) (layers *.Cu *.Mask) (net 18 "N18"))
  (pad "11" thru_hole circle (at 0 25.4 270) (size 1.8 1.8) (drill 0.8) (layers *.Cu *.Mask) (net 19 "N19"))
  (pad "12" thru_hole circle (at 0 27.94 270) (size 1.8 1.8) (drill 0.8) (layers *.Cu *.Mask) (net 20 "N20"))
  (pad "13" thru_hole circle (at 0 30.48 270) (size 1.8 1.8) (drill 0.8) (layers *.Cu *.Mask) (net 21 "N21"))
  (pad "14" thru_hole circle (at 0 33.02 270) (size 1.8 1.8) (drill 0.8) (layers *.Cu *.Mask) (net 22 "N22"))
  (pad "15" thru_hole circle (at 0 35.56 270) (size 1.8 1.8) (drill 0.8) (layers *.Cu *.Mask) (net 14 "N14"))
  (pad "16" thru_hole circle (at 15.24 35.56 270) (size 1.8 1.8) (drill 0.8) (layers *.Cu *.Mask) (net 6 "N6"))
  (pad "17" thru_hole circle (at 15.24 33.02 270) (size 1.8 1.8) (drill 0.8) (layers *.Cu *.Mask) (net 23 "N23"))
  (pad "18" thru_hole circle (at 15.24 30.48 270) (size 1.8 1.8) (drill 0.8) (layers *.Cu *.Mask) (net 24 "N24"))
  (pad "19" thru_hole circle (at 15.24 27.94 270) (size 1.8 1.8) (drill 0.8) (layers *.Cu *.Mask) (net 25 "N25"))
  (pad "20" thru_hole circle (at 15.24 25.4 270) (size 1.8 1.8) (drill 1) (layers *.Cu *.Mask) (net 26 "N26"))
  (pad "21" thru_hole circle (at 15.24 22.86 270) (size 1.8 1.8) (drill 0.8) (layers *.Cu *.Mask) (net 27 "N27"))
  (pad "22" thru_hole circle (at 15.24 20.32 270) (size 1.8 1.8) (drill 0.8) (layers *.Cu *.Mask) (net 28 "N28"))
  (pad "23" thru_hole circle (at 15.24 17.78 270) (size 1.8 1.8) (drill 0.8) (layers *.Cu *.Mask) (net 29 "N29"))
  (pad "24" thru_hole circle (at 15.24 15.24 270) (size 1.8 1.8) (drill 0.8) (layers *.Cu *.Mask) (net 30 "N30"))
  (pad "25" thru_hole circle (at 15.24 12.7 270) (size 1.8 1.8) (drill 0.8) (layers *.Cu *.Mask) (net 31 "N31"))
  (pad "26" thru_hole circle (at 15.24 10.16 270) (size 1.8 1.8) (drill 0.8) (layers *.Cu *.Mask) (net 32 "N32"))
  (pad "27" thru_hole circle (at 15.24 7.62 270) (size 1.8 1.8) (drill 0.8) (layers *.Cu *.Mask) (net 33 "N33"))
  (pad "28" thru_hole circle (at 15.24 5.08 270) (size 1.8 1.8) (drill 0.8) (layers *.Cu *.Mask) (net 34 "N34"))
  (pad "29" thru_hole circle (at 15.24 2.54 270) (size 1.8 1.8) (drill 0.8) (layers *.Cu *.Mask) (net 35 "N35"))
  (pad "30" thru_hole circle (at 15.24 0 270) (size 1.8 1.8) (drill 0.8) (layers *.Cu *.Mask) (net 1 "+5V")))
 (gr_rect (start 105.41 96.52) (end 128.41 119.52) (layer "F.SilkS") (width 0.15) (fill none))
 (gr_line (start 137.13 93.98) (end 137.13 156.21) (layer "Edge.Cuts") (width 0.1))
 (gr_line (start 137.13 156.21) (end 74.99 156.21) (layer "Edge.Cuts") (width 0.1))
 (gr_line (start 74.99 156.21) (end 74.99 93.98) (layer "Edge.Cuts") (width 0.1))
 (gr_line (start 74.99 93.98) (end 137.13 93.98) (layer "Edge.Cuts") (width 0.1))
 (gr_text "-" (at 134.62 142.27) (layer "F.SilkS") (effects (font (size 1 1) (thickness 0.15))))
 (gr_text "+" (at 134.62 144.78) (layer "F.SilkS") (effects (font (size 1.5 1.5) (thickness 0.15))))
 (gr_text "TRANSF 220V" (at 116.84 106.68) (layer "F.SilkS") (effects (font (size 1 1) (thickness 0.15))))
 (segment (start 116.84 137.17) (end 116.84 128.4) (width 1.4) (layer "B.Cu") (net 5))
 (segment (start 78.74 124.46) (end 83.82 124.46) (width 1.4) (layer "B.Cu") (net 5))
 (segment (start 119.42 125.77) (end 131.97 125.77) (width 1.4) (layer "B.Cu") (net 5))
 (segment (start 111.76 142.24) (end 119.38 142.24) (width 1.4) (layer "B.Cu") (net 5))
 (segment (start 132.08 142.21) (end 119.41 142.21) (width 1.4) (layer "B.Cu") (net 5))
 (segment (start 116.84 139.7) (end 116.84 137.17) (width 1.4) (layer "B.Cu") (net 5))
 (segment (start 109.22 139.7) (end 111.76 142.24) (width 1.4) (layer "B.Cu") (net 5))
 (segment (start 84.12 119.68) (end 90.57 113.23) (width 1.4) (layer "B.Cu") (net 5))
 (segment (start 83.82 124.46) (end 83.82 119.98) (width 1.4) (layer "B.Cu") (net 5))
 (segment (start 91.44 119.38) (end 84.42 119.38) (width 1.4) (layer "B.Cu") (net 5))
 (segment (start 83.82 119.98) (end 84.12 119.68) (width 1.4) (layer "B.Cu") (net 5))
 (segment (start 84.12 119.68) (end 84.42 119.38) (width 1.4) (layer "B.Cu") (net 5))
 (segment (start 109.22 129.54) (end 109.22 132.08) (width 1.4) (layer "B.Cu") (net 5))
 (segment (start 109.22 139.7) (end 109.22 132.08) (width 1.4) (layer "B.Cu") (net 5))
 (segment (start 116.84 128.4) (end 119.47 125.77) (width 1.4) (layer "B.Cu") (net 5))
 (segment (start 116.84 139.7) (end 119.38 142.24) (width 1.4) (layer "B.Cu") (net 5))
 (segment (start 83.82 124.46) (end 104.14 124.46) (width 1.4) (layer "B.Cu") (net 5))
 (segment (start 104.14 124.46) (end 109.22 129.54) (width 1.4) (layer "B.Cu") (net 5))
 (segment (start 95.25 130.81) (end 95.25 132.08) (width 1.4) (layer "B.Cu") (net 9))
 (segment (start 99.06 127) (end 95.25 130.81) (width 1.4) (layer "B.Cu") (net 9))
 (segment (start 88.9 137.16) (end 83.82 132.08) (width 1.4) (layer "B.Cu") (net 14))
 (segment (start 114.3 124.46) (end 116.84 121.92) (width 1.4) (layer "B.Cu") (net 1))
 (segment (start 129.54 144.78) (end 109.22 144.78) (width 1.4) (layer "B.Cu") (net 1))
 (segment (start 124.43 152.43) (end 124.43 149.89) (width 1.4) (layer "B.Cu") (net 1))
 (segment (start 106.68 132.08) (end 102.87 132.08) (width 1.4) (layer "B.Cu") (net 1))
 (segment (start 134.62 124.46) (end 134.62 143.51) (width 1.4) (layer "B.Cu") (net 1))
 (segment (start 109.22 144.78) (end 106.68 142.24) (width 1.4) (layer "B.Cu") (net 1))
 (segment (start 116.84 121.92) (end 132.08 121.92) (width 1.4) (layer "B.Cu") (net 1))
 (segment (start 134.62 143.51) (end 133.32 144.81) (width 1.4) (layer "B.Cu") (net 1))
 (segment (start 106.68 142.24) (end 106.68 132.08) (width 1.4) (layer "B.Cu") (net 1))
 (segment (start 129.54 144.78) (end 132.05 144.78) (width 1.4) (layer "B.Cu") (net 1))
 (segment (start 124.43 149.89) (end 129.54 144.78) (width 1.4) (layer "B.Cu") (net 1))
 (segment (start 133.32 144.81) (end 132.08 144.81) (width 1.4) (layer "B.Cu") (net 1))
 (segment (start 132.08 121.92) (end 134.62 124.46) (width 1.4) (layer "B.Cu") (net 1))
 (segment (start 78.74 127) (end 78.74 138.43) (width 1.4) (layer "B.Cu") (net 7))
 (segment (start 85.1 152.41) (end 78.74 146.05) (width 1.4) (layer "B.Cu") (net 6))
 (segment (start 88.9 152.41) (end 85.1 152.41) (width 1.4) (layer "B.Cu") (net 6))
 (segment (start 96.52 115.18) (end 96.52 114.3) (width 1.4) (layer "B.Cu") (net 11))
 (segment (start 86.36 109.22) (end 83.82 111.76) (width 1.4) (layer "B.Cu") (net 11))
 (segment (start 83.82 111.76) (end 82.55 111.76) (width 1.4) (layer "B.Cu") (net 11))
 (segment (start 96.52 114.3) (end 91.44 109.22) (width 1.4) (layer "B.Cu") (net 11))
 (segment (start 91.44 109.22) (end 86.36 109.22) (width 1.4) (layer "B.Cu") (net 11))
 (segment (start 119.38 130.86) (end 119.47 130.77) (width 1.4) (layer "B.Cu") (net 13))
 (segment (start 119.42 130.77) (end 131.97 130.77) (width 1.4) (layer "B.Cu") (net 13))
 (segment (start 119.38 137.17) (end 119.38 130.86) (width 1.4) (layer "B.Cu") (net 13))
 (segment (start 91.44 129.54) (end 88.9 127) (width 1.4) (layer "B.Cu") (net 8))
 (segment (start 91.44 132.08) (end 91.44 129.54) (width 1.4) (layer "B.Cu") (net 8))
 (segment (start 111.76 127) (end 111.76 124.46) (width 1.4) (layer "B.Cu") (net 2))
 (segment (start 114.3 129.54) (end 111.76 127) (width 1.4) (layer "B.Cu") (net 2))
 (segment (start 114.3 137.17) (end 114.3 129.54) (width 1.4) (layer "B.Cu") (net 2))
 (segment (start 111.76 137.17) (end 111.76 132.08) (width 1.4) (layer "B.Cu") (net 4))
 (segment (start 82.55 106.68) (end 82.55 105.41) (width 1.4) (layer "B.Cu") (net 10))
 (segment (start 86.98 100.98) (end 90.52 100.98) (width 1.4) (layer "B.Cu") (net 10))
 (segment (start 82.55 105.41) (end 86.98 100.98) (width 1.4) (layer "B.Cu") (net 10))
 (segment (start 104.14 119.38) (end 104.14 116.84) (width 1.4) (layer "B.Cu") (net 3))
 (segment (start 101.6 119.38) (end 104.14 119.38) (width 1.4) (layer "B.Cu") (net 3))
 (segment (start 102.57 115.27) (end 102.57 113.23) (width 1.4) (layer "B.Cu") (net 3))
 (segment (start 104.14 116.84) (end 102.57 115.27) (width 1.4) (layer "B.Cu") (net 3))
 (segment (start 109.22 124.46) (end 104.14 119.38) (width 1.4) (layer "B.Cu") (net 3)))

